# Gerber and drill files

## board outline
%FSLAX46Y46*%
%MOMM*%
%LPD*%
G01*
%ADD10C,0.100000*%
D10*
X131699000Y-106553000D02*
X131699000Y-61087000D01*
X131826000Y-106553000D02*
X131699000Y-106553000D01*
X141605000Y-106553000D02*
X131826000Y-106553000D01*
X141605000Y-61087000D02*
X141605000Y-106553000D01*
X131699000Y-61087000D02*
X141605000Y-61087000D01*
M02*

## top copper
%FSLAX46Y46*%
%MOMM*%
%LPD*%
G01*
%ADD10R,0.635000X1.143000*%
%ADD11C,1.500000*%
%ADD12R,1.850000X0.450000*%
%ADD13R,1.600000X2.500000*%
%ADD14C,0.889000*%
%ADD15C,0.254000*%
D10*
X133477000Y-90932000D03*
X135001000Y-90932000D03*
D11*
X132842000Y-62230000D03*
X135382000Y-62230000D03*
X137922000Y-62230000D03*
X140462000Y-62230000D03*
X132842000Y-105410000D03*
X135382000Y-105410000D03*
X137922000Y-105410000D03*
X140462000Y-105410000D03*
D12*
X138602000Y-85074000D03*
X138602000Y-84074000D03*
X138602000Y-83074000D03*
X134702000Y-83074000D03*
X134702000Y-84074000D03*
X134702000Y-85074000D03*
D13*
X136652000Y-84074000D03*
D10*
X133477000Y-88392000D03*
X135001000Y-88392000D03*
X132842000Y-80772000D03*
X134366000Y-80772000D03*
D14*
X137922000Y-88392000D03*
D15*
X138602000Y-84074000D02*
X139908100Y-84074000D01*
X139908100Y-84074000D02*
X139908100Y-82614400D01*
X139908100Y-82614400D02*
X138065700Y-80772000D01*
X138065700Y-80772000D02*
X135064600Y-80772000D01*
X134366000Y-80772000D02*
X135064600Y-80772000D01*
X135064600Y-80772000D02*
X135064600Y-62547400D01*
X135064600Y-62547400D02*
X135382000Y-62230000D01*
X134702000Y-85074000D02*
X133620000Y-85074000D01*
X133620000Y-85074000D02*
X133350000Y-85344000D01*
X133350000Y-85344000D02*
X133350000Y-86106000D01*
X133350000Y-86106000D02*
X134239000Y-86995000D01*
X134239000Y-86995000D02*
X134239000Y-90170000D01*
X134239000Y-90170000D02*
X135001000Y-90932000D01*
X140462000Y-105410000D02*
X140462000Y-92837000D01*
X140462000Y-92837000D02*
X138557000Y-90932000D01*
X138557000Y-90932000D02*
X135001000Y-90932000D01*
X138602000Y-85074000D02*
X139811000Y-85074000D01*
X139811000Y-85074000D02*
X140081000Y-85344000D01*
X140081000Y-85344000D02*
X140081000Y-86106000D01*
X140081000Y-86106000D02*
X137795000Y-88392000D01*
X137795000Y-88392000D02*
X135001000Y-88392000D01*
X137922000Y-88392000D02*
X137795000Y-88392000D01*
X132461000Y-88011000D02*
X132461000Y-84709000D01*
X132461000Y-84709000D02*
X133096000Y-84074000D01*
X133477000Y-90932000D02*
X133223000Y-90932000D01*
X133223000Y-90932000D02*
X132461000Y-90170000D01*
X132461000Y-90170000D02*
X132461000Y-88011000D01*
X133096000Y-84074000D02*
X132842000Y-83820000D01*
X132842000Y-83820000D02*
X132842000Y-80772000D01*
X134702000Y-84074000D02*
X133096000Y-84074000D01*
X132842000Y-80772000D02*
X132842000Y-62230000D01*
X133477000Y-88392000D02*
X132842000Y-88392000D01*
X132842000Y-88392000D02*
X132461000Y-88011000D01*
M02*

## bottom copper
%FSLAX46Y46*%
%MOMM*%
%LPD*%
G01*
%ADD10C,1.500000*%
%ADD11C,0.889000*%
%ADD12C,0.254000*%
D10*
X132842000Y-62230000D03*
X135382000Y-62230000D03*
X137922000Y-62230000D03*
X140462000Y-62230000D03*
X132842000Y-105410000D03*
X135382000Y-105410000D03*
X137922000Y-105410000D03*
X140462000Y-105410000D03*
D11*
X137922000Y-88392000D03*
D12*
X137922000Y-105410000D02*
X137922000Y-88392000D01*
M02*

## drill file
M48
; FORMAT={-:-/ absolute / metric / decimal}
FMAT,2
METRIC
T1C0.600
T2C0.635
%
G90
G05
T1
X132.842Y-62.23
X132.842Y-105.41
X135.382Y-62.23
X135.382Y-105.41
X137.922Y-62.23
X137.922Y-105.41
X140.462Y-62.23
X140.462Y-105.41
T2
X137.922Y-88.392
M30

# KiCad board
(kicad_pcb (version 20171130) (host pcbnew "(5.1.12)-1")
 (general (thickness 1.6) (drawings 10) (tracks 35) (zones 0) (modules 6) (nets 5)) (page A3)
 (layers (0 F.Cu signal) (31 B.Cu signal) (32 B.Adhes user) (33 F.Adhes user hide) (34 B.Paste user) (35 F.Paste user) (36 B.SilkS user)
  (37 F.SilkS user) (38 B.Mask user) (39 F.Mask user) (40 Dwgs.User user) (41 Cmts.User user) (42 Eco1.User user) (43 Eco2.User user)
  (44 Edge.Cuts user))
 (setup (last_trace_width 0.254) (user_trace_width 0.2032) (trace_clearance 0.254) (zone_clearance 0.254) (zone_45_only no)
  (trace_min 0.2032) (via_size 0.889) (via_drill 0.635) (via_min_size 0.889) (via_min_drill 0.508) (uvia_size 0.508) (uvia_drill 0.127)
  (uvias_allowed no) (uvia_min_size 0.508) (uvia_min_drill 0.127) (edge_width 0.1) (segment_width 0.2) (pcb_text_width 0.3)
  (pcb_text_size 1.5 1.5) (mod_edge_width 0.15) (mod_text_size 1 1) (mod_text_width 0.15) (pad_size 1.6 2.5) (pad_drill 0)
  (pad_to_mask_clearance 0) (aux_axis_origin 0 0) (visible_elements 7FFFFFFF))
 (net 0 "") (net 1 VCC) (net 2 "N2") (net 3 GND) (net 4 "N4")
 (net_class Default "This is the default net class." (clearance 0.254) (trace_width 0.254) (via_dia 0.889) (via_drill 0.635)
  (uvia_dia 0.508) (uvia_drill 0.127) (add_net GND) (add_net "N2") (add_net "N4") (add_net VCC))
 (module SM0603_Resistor (layer F.Cu) (at 134.239 90.932)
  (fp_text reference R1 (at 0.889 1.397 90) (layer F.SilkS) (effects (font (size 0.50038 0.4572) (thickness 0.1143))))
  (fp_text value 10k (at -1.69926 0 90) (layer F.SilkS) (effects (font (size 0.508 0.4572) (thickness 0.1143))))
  (pad 1 smd rect (at -0.762 0) (size 0.635 1.143) (layers F.Cu F.Paste F.Mask) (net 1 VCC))
  (pad 2 smd rect (at 0.762 0) (size 0.635 1.143) (layers F.Cu F.Paste F.Mask) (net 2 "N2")))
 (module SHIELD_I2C (layer F.Cu) (at 136.652 83.82)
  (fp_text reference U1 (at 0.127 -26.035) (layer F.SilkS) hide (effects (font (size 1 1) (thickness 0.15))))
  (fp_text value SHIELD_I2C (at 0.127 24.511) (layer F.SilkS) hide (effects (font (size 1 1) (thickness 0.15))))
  (pad 1 thru_hole circle (at -3.81 -21.59) (size 1.5 1.5) (drill 0.6) (layers *.Cu *.Mask F.SilkS) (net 1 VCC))
  (pad 2 thru_hole circle (at -1.27 -21.59) (size 1.5 1.5) (drill 0.6) (layers *.Cu *.Mask F.SilkS) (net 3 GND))
  (pad 3 thru_hole circle (at 1.27 -21.59) (size 1.5 1.5) (drill 0.6) (layers *.Cu *.Mask F.SilkS))
  (pad 4 thru_hole circle (at 3.81 -21.59) (size 1.5 1.5) (drill 0.6) (layers *.Cu *.Mask F.SilkS))
  (pad 5 thru_hole circle (at -3.81 21.59) (size 1.5 1.5) (drill 0.6) (layers *.Cu *.Mask F.SilkS))
  (pad 6 thru_hole circle (at -1.27 21.59) (size 1.5 1.5) (drill 0.6) (layers *.Cu *.Mask F.SilkS))
  (pad 7 thru_hole circle (at 1.27 21.59) (size 1.5 1.5) (drill 0.6) (layers *.Cu *.Mask F.SilkS) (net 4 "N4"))
  (pad 8 thru_hole circle (at 3.81 21.59) (size 1.5 1.5) (drill 0.6) (layers *.Cu *.Mask F.SilkS) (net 2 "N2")))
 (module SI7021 (layer F.Cu) (at 136.652 84.074 180) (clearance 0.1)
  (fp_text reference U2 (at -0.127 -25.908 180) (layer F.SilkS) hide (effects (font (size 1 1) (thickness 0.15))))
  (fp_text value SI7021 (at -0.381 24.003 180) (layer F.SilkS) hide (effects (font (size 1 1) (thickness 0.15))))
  (pad 1 smd rect (at -1.95 -1 180) (size 1.85 0.45) (layers F.Cu F.Paste F.Mask) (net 4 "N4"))
  (pad 2 smd rect (at -1.95 0 180) (size 1.85 0.45) (layers F.Cu F.Paste F.Mask) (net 3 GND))
  (pad 3 smd rect (at -1.95 1 180) (size 1.85 0.45) (layers F.Cu F.Paste F.Mask))
  (pad 4 smd rect (at 1.95 1 180) (size 1.85 0.45) (layers F.Cu F.Paste F.Mask))
  (pad 5 smd rect (at 1.95 0 180) (size 1.85 0.45) (layers F.Cu F.Paste F.Mask) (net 1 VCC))
  (pad 6 smd rect (at 1.95 -1 180) (size 1.85 0.45) (layers F.Cu F.Paste F.Mask) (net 2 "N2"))
  (pad 7 smd rect (at 0 0 180) (size 1.6 2.5) (layers F.Cu F.Paste F.Mask)))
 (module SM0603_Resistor (layer F.Cu) (at 134.239 88.392)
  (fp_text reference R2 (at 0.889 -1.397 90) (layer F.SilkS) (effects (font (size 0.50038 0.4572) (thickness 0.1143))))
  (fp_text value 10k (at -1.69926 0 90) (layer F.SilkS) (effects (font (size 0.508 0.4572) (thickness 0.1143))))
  (pad 1 smd rect (at -0.762 0) (size 0.635 1.143) (layers F.Cu F.Paste F.Mask) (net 1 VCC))
  (pad 2 smd rect (at 0.762 0) (size 0.635 1.143) (layers F.Cu F.Paste F.Mask) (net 4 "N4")))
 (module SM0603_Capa (layer F.Cu) (at 133.604 80.772)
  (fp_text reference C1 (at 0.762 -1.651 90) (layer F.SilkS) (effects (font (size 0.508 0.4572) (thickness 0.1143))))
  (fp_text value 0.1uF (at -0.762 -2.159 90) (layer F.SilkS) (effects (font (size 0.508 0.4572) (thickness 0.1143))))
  (pad 1 smd rect (at -0.762 0) (size 0.635 1.143) (layers F.Cu F.Paste F.Mask) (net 1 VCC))
  (pad 2 smd rect (at 0.762 0) (size 0.635 1.143) (layers F.Cu F.Paste F.Mask) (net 3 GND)))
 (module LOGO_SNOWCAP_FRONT (layer F.Cu) (at 138.811 71.501 90)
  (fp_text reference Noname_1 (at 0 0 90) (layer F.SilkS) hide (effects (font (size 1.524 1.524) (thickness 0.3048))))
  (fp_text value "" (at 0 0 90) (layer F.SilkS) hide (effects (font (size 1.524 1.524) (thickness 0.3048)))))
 (gr_line (start 131.699 106.553) (end 131.699 61.087) (angle 90) (layer Edge.Cuts) (width 0.1))
 (gr_line (start 131.826 106.553) (end 131.699 106.553) (angle 90) (layer Edge.Cuts) (width 0.1))
 (gr_line (start 141.605 106.553) (end 131.826 106.553) (angle 90) (layer Edge.Cuts) (width 0.1))
 (gr_line (start 141.605 61.087) (end 141.605 106.553) (angle 90) (layer Edge.Cuts) (width 0.1))
 (gr_line (start 131.699 61.087) (end 141.605 61.087) (angle 90) (layer Edge.Cuts) (width 0.1))
 (segment (start 138.602 84.074) (end 139.9081 84.074) (width 0.254) (layer F.Cu) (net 3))
 (segment (start 139.9081 84.074) (end 139.9081 82.6144) (width 0.254) (layer F.Cu) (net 3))
 (segment (start 139.9081 82.6144) (end 138.0657 80.772) (width 0.254) (layer F.Cu) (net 3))
 (segment (start 138.0657 80.772) (end 135.0646 80.772) (width 0.254) (layer F.Cu) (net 3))
 (segment (start 134.366 80.772) (end 135.0646 80.772) (width 0.254) (layer F.Cu) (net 3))
 (segment (start 135.0646 80.772) (end 135.0646 62.5474) (width 0.254) (layer F.Cu) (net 3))
 (segment (start 135.0646 62.5474) (end 135.382 62.23) (width 0.254) (layer F.Cu) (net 3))
 (segment (start 134.702 85.074) (end 133.62 85.074) (width 0.254) (layer F.Cu) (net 2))
 (segment (start 133.62 85.074) (end 133.35 85.344) (width 0.254) (layer F.Cu) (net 2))
 (segment (start 133.35 85.344) (end 133.35 86.106) (width 0.254) (layer F.Cu) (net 2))
 (segment (start 133.35 86.106) (end 134.239 86.995) (width 0.254) (layer F.Cu) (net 2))
 (segment (start 134.239 86.995) (end 134.239 90.17) (width 0.254) (layer F.Cu) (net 2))
 (segment (start 134.239 90.17) (end 135.001 90.932) (width 0.254) (layer F.Cu) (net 2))
 (segment (start 140.462 105.41) (end 140.462 92.837) (width 0.254) (layer F.Cu) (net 2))
 (segment (start 140.462 92.837) (end 138.557 90.932) (width 0.254) (layer F.Cu) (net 2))
 (segment (start 138.557 90.932) (end 135.001 90.932) (width 0.254) (layer F.Cu) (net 2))
 (segment (start 138.602 85.074) (end 139.811 85.074) (width 0.254) (layer F.Cu) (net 4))
 (segment (start 139.811 85.074) (end 140.081 85.344) (width 0.254) (layer F.Cu) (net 4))
 (segment (start 140.081 85.344) (end 140.081 86.106) (width 0.254) (layer F.Cu) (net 4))
 (segment (start 140.081 86.106) (end 137.795 88.392) (width 0.254) (layer F.Cu) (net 4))
 (segment (start 137.795 88.392) (end 135.001 88.392) (width 0.254) (layer F.Cu) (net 4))
 (segment (start 137.922 88.392) (end 137.795 88.392) (width 0.254) (layer F.Cu) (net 4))
 (segment (start 137.922 105.41) (end 137.922 88.392) (width 0.254) (layer B.Cu) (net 4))
 (via (at 137.922 88.392) (size 0.889) (layers F.Cu B.Cu) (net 4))
 (segment (start 132.461 88.011) (end 132.461 84.709) (width 0.254) (layer F.Cu) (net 1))
 (segment (start 132.461 84.709) (end 133.096 84.074) (width 0.254) (layer F.Cu) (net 1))
 (segment (start 133.477 90.932) (end 133.223 90.932) (width 0.254) (layer F.Cu) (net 1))
 (segment (start 133.223 90.932) (end 132.461 90.17) (width 0.254) (layer F.Cu) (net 1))
 (segment (start 132.461 90.17) (end 132.461 88.011) (width 0.254) (layer F.Cu) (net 1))
 (segment (start 133.096 84.074) (end 132.842 83.82) (width 0.254) (layer F.Cu) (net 1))
 (segment (start 132.842 83.82) (end 132.842 80.772) (width 0.254) (layer F.Cu) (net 1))
 (segment (start 134.702 84.074) (end 133.096 84.074) (width 0.254) (layer F.Cu) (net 1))
 (segment (start 132.842 80.772) (end 132.842 62.23) (width 0.254) (layer F.Cu) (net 1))
 (segment (start 133.477 88.392) (end 132.842 88.392) (width 0.254) (layer F.Cu) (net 1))
 (segment (start 132.842 88.392) (end 132.461 88.011) (width 0.254) (layer F.Cu) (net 1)))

